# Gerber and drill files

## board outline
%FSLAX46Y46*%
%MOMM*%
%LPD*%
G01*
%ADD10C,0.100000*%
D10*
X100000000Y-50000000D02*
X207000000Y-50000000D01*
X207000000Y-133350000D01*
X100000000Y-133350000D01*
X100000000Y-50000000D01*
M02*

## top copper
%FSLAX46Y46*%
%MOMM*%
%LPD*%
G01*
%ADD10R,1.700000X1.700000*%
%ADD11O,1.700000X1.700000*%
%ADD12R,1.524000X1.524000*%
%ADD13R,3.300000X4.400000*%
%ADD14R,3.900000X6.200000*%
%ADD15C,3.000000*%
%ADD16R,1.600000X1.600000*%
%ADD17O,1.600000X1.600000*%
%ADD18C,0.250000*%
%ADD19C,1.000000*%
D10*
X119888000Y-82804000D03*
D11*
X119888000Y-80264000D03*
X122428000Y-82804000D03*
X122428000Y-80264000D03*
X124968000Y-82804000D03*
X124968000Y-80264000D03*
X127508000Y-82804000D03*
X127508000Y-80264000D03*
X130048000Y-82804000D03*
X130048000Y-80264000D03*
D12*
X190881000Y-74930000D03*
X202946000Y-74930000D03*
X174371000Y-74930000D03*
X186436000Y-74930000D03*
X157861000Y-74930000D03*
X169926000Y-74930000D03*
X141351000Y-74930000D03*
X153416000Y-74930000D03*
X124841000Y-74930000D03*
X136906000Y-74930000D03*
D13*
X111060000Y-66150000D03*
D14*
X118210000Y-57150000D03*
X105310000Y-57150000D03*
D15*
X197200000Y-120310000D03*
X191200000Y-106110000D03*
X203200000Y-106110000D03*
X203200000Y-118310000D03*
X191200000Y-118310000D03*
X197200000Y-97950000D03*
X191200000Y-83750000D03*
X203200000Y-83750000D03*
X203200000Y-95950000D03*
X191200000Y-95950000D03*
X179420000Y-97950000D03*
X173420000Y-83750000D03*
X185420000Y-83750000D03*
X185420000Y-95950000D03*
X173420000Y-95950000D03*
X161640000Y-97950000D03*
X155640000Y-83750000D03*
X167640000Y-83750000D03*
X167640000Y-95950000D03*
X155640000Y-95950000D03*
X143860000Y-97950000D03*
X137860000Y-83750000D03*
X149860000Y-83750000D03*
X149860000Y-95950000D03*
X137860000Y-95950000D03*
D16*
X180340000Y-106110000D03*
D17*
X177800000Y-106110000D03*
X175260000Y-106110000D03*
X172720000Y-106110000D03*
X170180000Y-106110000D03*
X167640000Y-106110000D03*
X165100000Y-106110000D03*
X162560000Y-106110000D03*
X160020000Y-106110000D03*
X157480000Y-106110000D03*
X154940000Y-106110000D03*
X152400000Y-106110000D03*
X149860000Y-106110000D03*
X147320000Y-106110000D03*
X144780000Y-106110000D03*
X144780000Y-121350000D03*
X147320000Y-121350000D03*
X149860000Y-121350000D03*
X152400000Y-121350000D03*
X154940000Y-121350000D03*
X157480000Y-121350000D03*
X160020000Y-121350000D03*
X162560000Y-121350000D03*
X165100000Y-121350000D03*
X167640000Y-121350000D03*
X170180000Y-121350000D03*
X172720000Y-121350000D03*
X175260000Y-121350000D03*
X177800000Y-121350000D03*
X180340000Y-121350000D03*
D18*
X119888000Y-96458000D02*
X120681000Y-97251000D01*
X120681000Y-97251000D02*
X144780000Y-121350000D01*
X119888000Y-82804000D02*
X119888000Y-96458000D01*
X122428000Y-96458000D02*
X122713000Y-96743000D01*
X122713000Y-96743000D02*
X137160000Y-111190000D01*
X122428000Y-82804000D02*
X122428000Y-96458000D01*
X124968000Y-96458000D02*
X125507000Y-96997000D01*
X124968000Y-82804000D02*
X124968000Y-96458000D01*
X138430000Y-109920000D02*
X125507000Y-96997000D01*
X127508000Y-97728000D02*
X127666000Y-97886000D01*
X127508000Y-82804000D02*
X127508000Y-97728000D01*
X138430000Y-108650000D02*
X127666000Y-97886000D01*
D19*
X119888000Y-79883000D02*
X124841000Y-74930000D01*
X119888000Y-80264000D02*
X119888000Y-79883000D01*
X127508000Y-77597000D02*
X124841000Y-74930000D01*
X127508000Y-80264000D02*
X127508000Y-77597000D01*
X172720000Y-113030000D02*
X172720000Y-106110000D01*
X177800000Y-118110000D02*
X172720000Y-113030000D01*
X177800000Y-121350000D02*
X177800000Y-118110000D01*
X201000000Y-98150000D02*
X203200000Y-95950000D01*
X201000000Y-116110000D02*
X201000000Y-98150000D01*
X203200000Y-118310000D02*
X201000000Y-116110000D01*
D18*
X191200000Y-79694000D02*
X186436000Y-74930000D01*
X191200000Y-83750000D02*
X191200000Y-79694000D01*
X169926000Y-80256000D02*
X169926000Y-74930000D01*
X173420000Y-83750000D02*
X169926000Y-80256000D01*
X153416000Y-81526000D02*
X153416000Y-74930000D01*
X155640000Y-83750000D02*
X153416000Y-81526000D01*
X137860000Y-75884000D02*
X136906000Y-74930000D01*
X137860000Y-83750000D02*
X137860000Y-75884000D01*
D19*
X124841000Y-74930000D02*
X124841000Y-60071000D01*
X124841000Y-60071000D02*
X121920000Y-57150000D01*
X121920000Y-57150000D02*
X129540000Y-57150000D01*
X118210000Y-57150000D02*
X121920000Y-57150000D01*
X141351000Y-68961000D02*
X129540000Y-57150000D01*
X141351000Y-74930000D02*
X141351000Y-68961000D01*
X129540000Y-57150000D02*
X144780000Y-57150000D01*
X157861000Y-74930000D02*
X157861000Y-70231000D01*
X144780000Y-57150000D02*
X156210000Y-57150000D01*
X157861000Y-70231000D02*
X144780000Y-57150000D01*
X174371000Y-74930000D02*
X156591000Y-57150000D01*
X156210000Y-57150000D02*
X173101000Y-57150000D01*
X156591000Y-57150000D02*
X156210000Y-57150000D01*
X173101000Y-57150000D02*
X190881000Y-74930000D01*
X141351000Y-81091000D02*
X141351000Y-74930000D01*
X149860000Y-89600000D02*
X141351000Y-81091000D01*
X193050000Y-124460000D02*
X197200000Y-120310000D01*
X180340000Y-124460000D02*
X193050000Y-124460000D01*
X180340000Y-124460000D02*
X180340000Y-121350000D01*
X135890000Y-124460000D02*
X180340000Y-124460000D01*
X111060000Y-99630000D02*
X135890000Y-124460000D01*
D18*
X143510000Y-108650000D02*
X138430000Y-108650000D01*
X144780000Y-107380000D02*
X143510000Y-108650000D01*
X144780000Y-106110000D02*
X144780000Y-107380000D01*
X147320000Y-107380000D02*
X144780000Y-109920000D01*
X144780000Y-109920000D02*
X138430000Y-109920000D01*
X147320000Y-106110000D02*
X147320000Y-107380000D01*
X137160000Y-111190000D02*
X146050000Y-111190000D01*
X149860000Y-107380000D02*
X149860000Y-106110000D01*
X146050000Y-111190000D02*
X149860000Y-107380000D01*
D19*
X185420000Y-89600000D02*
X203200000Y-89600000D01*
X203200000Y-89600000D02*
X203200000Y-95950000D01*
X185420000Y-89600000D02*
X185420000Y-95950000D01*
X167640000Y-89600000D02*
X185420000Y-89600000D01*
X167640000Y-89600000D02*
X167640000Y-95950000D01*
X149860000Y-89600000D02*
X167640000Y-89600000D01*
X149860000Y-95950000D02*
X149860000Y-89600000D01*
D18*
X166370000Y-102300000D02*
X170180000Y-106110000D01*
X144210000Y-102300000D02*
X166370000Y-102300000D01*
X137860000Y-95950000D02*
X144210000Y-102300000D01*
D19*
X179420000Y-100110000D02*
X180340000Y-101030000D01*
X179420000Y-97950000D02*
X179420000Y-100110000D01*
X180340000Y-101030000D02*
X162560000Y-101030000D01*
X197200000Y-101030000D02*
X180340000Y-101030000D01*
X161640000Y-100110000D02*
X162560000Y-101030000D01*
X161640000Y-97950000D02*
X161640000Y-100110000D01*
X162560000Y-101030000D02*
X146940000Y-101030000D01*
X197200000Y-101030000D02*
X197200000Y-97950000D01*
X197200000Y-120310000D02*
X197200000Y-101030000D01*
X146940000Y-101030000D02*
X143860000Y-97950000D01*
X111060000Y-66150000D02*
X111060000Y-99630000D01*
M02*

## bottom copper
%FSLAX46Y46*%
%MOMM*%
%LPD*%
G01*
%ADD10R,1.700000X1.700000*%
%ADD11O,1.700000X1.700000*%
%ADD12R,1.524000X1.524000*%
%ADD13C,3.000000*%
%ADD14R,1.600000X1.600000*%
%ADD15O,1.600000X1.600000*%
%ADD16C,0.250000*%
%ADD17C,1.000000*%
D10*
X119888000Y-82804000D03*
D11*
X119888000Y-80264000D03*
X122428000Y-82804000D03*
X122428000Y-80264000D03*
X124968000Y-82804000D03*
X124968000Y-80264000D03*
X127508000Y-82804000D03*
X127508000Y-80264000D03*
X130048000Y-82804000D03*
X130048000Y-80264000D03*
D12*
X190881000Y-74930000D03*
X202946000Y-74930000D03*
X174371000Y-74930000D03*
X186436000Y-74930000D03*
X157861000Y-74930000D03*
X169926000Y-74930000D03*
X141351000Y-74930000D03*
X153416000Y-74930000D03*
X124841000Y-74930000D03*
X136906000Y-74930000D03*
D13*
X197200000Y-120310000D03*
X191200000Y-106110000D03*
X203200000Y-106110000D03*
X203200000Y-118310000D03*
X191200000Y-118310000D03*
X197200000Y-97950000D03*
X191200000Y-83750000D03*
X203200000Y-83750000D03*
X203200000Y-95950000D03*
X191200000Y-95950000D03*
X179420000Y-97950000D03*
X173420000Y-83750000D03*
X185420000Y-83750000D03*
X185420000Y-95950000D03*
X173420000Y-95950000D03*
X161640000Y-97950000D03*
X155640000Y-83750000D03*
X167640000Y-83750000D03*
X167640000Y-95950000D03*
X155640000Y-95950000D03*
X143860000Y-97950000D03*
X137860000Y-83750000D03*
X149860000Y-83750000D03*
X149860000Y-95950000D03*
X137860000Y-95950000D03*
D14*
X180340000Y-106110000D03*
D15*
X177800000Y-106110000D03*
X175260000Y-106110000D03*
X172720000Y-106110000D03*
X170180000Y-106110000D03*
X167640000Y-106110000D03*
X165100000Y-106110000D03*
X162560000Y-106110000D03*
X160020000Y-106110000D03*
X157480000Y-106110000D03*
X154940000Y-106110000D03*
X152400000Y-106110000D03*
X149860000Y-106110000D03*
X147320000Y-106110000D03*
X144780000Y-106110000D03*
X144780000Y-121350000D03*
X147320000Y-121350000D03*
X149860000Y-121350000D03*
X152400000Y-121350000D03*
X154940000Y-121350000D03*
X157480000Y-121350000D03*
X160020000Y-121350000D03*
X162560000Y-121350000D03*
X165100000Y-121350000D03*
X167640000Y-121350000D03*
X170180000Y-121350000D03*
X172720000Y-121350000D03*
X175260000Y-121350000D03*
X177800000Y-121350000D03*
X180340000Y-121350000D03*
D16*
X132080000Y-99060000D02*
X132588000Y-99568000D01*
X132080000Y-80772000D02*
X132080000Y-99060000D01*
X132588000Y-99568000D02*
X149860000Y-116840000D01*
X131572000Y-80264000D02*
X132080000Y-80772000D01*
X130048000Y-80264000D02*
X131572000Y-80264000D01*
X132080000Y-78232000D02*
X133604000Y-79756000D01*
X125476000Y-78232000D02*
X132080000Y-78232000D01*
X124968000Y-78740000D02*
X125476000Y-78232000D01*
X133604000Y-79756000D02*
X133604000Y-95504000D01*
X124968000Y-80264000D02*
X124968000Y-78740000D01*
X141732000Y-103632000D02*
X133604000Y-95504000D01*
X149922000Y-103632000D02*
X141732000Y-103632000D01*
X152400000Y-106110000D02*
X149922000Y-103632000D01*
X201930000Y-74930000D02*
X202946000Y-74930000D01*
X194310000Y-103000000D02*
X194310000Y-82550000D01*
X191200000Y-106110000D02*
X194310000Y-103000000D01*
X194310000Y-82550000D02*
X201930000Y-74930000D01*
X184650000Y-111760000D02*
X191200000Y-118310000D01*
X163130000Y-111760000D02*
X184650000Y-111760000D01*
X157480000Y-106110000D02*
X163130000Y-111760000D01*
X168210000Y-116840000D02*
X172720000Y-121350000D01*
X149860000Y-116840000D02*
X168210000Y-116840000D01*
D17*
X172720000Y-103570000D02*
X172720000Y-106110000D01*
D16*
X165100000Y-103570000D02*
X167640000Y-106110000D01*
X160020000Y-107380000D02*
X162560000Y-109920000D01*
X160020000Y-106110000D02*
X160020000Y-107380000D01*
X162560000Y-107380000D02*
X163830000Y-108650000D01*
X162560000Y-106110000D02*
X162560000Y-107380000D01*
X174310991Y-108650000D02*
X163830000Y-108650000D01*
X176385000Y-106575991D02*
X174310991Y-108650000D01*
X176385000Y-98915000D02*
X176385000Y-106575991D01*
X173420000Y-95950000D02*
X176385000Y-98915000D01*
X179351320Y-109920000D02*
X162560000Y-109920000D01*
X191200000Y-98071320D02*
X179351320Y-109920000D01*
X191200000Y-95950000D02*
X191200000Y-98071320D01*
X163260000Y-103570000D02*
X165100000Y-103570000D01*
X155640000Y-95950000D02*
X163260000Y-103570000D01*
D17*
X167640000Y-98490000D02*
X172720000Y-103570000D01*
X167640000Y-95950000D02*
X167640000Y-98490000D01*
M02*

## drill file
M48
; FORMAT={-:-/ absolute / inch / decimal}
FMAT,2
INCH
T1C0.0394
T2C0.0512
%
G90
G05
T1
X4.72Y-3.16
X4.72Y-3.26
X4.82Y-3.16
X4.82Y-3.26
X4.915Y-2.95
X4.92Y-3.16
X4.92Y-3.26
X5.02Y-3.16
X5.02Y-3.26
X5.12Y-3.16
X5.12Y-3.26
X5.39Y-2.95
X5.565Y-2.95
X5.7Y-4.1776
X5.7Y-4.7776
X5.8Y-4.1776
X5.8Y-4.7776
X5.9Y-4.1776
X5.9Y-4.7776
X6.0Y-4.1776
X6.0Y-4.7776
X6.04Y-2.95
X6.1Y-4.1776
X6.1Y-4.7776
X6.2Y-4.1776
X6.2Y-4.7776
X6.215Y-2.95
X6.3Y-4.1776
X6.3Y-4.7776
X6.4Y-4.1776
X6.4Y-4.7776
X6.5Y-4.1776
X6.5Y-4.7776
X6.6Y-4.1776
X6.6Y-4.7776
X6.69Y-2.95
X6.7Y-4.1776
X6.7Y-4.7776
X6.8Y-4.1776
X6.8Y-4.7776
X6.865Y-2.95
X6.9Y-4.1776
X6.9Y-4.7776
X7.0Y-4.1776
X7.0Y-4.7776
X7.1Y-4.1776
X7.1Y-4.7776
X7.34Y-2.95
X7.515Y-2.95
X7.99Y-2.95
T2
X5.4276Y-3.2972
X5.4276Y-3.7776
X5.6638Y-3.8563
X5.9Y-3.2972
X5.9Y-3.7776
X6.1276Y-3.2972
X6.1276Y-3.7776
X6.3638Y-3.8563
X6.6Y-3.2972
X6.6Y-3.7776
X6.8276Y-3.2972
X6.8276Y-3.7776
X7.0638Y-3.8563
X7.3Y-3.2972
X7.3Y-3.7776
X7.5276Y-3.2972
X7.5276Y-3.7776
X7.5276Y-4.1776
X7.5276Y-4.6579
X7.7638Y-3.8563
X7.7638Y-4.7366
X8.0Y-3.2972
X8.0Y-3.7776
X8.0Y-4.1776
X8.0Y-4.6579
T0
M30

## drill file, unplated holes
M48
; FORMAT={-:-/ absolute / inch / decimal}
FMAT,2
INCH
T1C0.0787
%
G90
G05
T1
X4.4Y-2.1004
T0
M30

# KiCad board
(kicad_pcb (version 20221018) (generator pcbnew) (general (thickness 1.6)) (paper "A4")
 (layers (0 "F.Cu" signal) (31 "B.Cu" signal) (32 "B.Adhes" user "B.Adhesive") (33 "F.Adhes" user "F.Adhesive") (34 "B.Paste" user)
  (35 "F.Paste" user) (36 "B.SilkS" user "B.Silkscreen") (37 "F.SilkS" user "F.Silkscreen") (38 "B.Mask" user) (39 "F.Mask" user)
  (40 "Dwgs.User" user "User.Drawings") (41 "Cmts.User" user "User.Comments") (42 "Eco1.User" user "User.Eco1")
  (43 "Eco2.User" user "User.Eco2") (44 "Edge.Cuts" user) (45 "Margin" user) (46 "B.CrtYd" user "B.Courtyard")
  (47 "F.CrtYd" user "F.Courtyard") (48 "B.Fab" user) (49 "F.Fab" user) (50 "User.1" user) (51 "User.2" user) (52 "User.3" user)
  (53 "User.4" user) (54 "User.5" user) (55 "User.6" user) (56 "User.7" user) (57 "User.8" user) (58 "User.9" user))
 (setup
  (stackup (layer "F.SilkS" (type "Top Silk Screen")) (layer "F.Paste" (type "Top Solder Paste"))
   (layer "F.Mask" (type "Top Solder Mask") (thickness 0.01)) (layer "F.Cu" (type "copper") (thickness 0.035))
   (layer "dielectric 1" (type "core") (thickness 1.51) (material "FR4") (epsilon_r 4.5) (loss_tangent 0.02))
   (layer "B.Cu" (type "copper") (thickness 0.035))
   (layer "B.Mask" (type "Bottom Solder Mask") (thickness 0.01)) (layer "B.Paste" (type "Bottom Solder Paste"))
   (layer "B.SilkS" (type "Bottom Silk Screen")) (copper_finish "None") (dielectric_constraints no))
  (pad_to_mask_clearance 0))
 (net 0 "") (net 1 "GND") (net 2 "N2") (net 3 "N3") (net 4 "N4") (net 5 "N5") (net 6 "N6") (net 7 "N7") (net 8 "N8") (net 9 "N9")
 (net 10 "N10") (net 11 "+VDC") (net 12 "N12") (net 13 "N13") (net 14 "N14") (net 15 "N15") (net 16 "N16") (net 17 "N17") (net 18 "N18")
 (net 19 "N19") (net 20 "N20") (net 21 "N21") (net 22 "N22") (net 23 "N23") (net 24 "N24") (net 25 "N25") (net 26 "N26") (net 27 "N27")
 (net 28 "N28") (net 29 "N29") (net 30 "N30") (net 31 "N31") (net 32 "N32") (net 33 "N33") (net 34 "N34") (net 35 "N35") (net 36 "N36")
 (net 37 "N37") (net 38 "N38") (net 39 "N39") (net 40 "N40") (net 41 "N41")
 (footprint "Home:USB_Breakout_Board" (layer "F.Cu") (at 196.85 62.23)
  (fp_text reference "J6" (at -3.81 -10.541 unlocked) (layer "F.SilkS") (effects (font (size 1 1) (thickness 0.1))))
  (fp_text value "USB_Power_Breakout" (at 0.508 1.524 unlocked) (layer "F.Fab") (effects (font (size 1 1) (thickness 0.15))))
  (pad "1" thru_hole rect (at -5.969 12.7) (size 1.524 1.524) (drill 1) (layers "*.Cu" "*.Mask") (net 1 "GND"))
  (pad "2" thru_hole rect (at 6.096 12.7) (size 1.524 1.524) (drill 1) (layers "*.Cu" "*.Mask") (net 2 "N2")))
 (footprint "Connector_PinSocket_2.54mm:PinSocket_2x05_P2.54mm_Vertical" (layer "F.Cu") (at 119.888 80.264 90)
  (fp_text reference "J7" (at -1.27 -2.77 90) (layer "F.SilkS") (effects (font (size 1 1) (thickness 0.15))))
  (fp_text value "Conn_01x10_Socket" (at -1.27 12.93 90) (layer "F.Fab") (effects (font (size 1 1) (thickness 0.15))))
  (pad "1" thru_hole rect (at -2.54 0 90) (size 1.7 1.7) (drill 1) (layers "*.Cu" "*.Mask") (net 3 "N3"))
  (pad "2" thru_hole oval (at 0 0 90) (size 1.7 1.7) (drill 1) (layers "*.Cu" "*.Mask") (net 1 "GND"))
  (pad "3" thru_hole oval (at -2.54 2.54 90) (size 1.7 1.7) (drill 1) (layers "*.Cu" "*.Mask") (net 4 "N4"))
  (pad "4" thru_hole oval (at 0 2.54 90) (size 1.7 1.7) (drill 1) (layers "*.Cu" "*.Mask") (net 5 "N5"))
  (pad "5" thru_hole oval (at -2.54 5.08 90) (size 1.7 1.7) (drill 1) (layers "*.Cu" "*.Mask") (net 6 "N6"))
  (pad "6" thru_hole oval (at 0 5.08 90) (size 1.7 1.7) (drill 1) (layers "*.Cu" "*.Mask") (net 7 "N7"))
  (pad "7" thru_hole oval (at -2.54 7.62 90) (size 1.7 1.7) (drill 1) (layers "*.Cu" "*.Mask") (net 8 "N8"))
  (pad "8" thru_hole oval (at 0 7.62 90) (size 1.7 1.7) (drill 1) (layers "*.Cu" "*.Mask") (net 1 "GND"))
  (pad "9" thru_hole oval (at -2.54 10.16 90) (size 1.7 1.7) (drill 1) (layers "*.Cu" "*.Mask") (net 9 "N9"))
  (pad "10" thru_hole oval (at 0 10.16 90) (size 1.7 1.7) (drill 1) (layers "*.Cu" "*.Mask") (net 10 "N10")))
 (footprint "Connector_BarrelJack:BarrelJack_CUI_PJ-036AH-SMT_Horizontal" (layer "F.Cu") (at 111.76 60.35 180)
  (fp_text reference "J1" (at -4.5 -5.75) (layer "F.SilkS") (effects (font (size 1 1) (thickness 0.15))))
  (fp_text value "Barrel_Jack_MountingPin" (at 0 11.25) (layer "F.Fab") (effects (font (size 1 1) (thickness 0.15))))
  (pad "" np_thru_hole circle (at 0 7 180) (size 2 2) (drill 2) (layers "*.Cu" "*.Mask"))
  (pad "1" smd rect (at 0.7 -5.8 180) (size 3.3 4.4) (layers "F.Cu" "F.Paste" "F.Mask") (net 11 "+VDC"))
  (pad "2" smd rect (at -6.45 3.2 180) (size 3.9 6.2) (layers "F.Cu" "F.Paste" "F.Mask") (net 1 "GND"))
  (pad "3" smd rect (at 6.45 3.2 180) (size 3.9 6.2) (layers "F.Cu" "F.Paste" "F.Mask")))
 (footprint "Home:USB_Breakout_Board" (layer "F.Cu") (at 180.34 62.23)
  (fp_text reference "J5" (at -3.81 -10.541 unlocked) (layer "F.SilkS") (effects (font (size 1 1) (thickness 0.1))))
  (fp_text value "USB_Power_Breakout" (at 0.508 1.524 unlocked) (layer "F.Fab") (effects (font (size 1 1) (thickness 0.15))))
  (pad "1" thru_hole rect (at -5.969 12.7) (size 1.524 1.524) (drill 1) (layers "*.Cu" "*.Mask") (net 1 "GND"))
  (pad "2" thru_hole rect (at 6.096 12.7) (size 1.524 1.524) (drill 1) (layers "*.Cu" "*.Mask") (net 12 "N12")))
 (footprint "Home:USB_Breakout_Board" (layer "F.Cu") (at 130.81 62.23)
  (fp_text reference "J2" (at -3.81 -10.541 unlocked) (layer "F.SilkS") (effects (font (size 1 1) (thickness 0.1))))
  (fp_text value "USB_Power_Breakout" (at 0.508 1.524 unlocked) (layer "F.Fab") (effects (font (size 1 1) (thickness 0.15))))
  (pad "1" thru_hole rect (at -5.969 12.7) (size 1.524 1.524) (drill 1) (layers "*.Cu" "*.Mask") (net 1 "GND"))
  (pad "2" thru_hole rect (at 6.096 12.7) (size 1.524 1.524) (drill 1) (layers "*.Cu" "*.Mask") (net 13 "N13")))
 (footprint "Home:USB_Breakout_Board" (layer "F.Cu") (at 147.32 62.23)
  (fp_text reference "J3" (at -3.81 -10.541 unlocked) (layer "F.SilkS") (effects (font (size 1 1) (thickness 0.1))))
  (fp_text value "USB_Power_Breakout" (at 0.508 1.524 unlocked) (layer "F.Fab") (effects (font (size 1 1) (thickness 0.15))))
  (pad "1" thru_hole rect (at -5.969 12.7) (size 1.524 1.524) (drill 1) (layers "*.Cu" "*.Mask") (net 1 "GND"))
  (pad "2" thru_hole rect (at 6.096 12.7) (size 1.524 1.524) (drill 1) (layers "*.Cu" "*.Mask") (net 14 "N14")))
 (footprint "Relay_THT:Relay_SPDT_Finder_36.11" (layer "F.Cu") (at 161.64 97.95 90)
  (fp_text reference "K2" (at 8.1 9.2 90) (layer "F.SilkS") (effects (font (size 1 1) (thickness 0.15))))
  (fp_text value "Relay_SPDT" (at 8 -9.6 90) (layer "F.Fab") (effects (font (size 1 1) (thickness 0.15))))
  (pad "11" thru_hole circle (at 0 0 90) (size 3 3) (drill 1.3) (layers "*.Cu" "*.Mask") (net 11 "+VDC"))
  (pad "12" thru_hole circle (at 14.2 -6 90) (size 3 3) (drill 1.3) (layers "*.Cu" "*.Mask") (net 14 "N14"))
  (pad "14" thru_hole circle (at 14.2 6 90) (size 3 3) (drill 1.3) (layers "*.Cu" "*.Mask") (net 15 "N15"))
  (pad "A1" thru_hole circle (at 2 6 90) (size 3 3) (drill 1.3) (layers "*.Cu" "*.Mask") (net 1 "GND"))
  (pad "A2" thru_hole circle (at 2 -6 90) (size 3 3) (drill 1.3) (layers "*.Cu" "*.Mask") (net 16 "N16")))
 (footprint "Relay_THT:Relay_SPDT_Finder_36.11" (layer "F.Cu") (at 179.42 97.95 90)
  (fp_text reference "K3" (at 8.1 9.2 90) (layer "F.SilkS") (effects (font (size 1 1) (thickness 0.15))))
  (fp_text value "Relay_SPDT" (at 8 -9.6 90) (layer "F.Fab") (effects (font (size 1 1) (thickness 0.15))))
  (pad "11" thru_hole circle (at 0 0 90) (size 3 3) (drill 1.3) (layers "*.Cu" "*.Mask") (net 11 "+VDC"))
  (pad "12" thru_hole circle (at 14.2 -6 90) (size 3 3) (drill 1.3) (layers "*.Cu" "*.Mask") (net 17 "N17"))
  (pad "14" thru_hole circle (at 14.2 6 90) (size 3 3) (drill 1.3) (layers "*.Cu" "*.Mask") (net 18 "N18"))
  (pad "A1" thru_hole circle (at 2 6 90) (size 3 3) (drill 1.3) (layers "*.Cu" "*.Mask") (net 1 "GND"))
  (pad "A2" thru_hole circle (at 2 -6 90) (size 3 3) (drill 1.3) (layers "*.Cu" "*.Mask") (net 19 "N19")))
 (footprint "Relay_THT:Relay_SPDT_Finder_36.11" (layer "F.Cu") (at 197.2 97.95 90)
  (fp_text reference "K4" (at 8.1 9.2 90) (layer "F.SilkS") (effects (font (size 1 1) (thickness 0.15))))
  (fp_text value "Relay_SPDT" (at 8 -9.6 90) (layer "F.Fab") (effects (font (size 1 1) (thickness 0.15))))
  (pad "11" thru_hole circle (at 0 0 90) (size 3 3) (drill 1.3) (layers "*.Cu" "*.Mask") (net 11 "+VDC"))
  (pad "12" thru_hole circle (at 14.2 -6 90) (size 3 3) (drill 1.3) (layers "*.Cu" "*.Mask") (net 12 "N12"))
  (pad "14" thru_hole circle (at 14.2 6 90) (size 3 3) (drill 1.3) (layers "*.Cu" "*.Mask") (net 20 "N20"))
  (pad "A1" thru_hole circle (at 2 6 90) (size 3 3) (drill 1.3) (layers "*.Cu" "*.Mask") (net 1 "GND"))
  (pad "A2" thru_hole circle (at 2 -6 90) (size 3 3) (drill 1.3) (layers "*.Cu" "*.Mask") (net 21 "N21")))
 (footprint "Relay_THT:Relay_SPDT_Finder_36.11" (layer "F.Cu") (at 143.86 97.95 90)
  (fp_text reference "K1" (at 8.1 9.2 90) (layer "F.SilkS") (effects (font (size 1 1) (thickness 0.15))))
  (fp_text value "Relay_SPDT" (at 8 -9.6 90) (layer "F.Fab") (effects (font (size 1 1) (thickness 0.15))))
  (pad "11" thru_hole circle (at 0 0 90) (size 3 3) (drill 1.3) (layers "*.Cu" "*.Mask") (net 11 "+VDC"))
  (pad "12" thru_hole circle (at 14.2 -6 90) (size 3 3) (drill 1.3) (layers "*.Cu" "*.Mask") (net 13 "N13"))
  (pad "14" thru_hole circle (at 14.2 6 90) (size 3 3) (drill 1.3) (layers "*.Cu" "*.Mask") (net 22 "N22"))
  (pad "A1" thru_hole circle (at 2 6 90) (size 3 3) (drill 1.3) (layers "*.Cu" "*.Mask") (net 1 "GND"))
  (pad "A2" thru_hole circle (at 2 -6 90) (size 3 3) (drill 1.3) (layers "*.Cu" "*.Mask") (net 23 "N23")))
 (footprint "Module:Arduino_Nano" (layer "F.Cu") (at 180.34 106.11 -90)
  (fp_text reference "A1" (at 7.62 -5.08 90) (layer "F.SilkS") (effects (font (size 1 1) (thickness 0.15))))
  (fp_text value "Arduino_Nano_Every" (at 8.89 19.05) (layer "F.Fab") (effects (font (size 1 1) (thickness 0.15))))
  (pad "1" thru_hole rect (at 0 0 270) (size 1.6 1.6) (drill 1) (layers "*.Cu" "*.Mask") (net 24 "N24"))
  (pad "2" thru_hole oval (at 0 2.54 270) (size 1.6 1.6) (drill 1) (layers "*.Cu" "*.Mask") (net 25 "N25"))
  (pad "3" thru_hole oval (at 0 5.08 270) (size 1.6 1.6) (drill 1) (layers "*.Cu" "*.Mask") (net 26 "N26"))
  (pad "4" thru_hole oval (at 0 7.62 270) (size 1.6 1.6) (drill 1) (layers "*.Cu" "*.Mask") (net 1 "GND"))
  (pad "5" thru_hole oval (at 0 10.16 270) (size 1.6 1.6) (drill 1) (layers "*.Cu" "*.Mask") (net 23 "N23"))
  (pad "6" thru_hole oval (at 0 12.7 270) (size 1.6 1.6) (drill 1) (layers "*.Cu" "*.Mask") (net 16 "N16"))
  (pad "7" thru_hole oval (at 0 15.24 270) (size 1.6 1.6) (drill 1) (layers "*.Cu" "*.Mask") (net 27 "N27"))
  (pad "8" thru_hole oval (at 0 17.78 270) (size 1.6 1.6) (drill 1) (layers "*.Cu" "*.Mask") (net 19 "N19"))
  (pad "9" thru_hole oval (at 0 20.32 270) (size 1.6 1.6) (drill 1) (layers "*.Cu" "*.Mask") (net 21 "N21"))
  (pad "10" thru_hole oval (at 0 22.86 270) (size 1.6 1.6) (drill 1) (layers "*.Cu" "*.Mask") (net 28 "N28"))
  (pad "11" thru_hole oval (at 0 25.4 270) (size 1.6 1.6) (drill 1) (layers "*.Cu" "*.Mask") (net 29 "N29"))
  (pad "12" thru_hole oval (at 0 27.94 270) (size 1.6 1.6) (drill 1) (layers "*.Cu" "*.Mask") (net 7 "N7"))
  (pad "13" thru_hole oval (at 0 30.48 270) (size 1.6 1.6) (drill 1) (layers "*.Cu" "*.Mask") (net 4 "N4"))
  (pad "14" thru_hole oval (at 0 33.02 270) (size 1.6 1.6) (drill 1) (layers "*.Cu" "*.Mask") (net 6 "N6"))
  (pad "15" thru_hole oval (at 0 35.56 270) (size 1.6 1.6) (drill 1) (layers "*.Cu" "*.Mask") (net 8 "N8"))
  (pad "16" thru_hole oval (at 15.24 35.56 270) (size 1.6 1.6) (drill 1) (layers "*.Cu" "*.Mask") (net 3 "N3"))
  (pad "17" thru_hole oval (at 15.24 33.02 270) (size 1.6 1.6) (drill 1) (layers "*.Cu" "*.Mask") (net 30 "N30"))
  (pad "18" thru_hole oval (at 15.24 30.48 270) (size 1.6 1.6) (drill 1) (layers "*.Cu" "*.Mask") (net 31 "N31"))
  (pad "19" thru_hole oval (at 15.24 27.94 270) (size 1.6 1.6) (drill 1) (layers "*.Cu" "*.Mask") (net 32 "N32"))
  (pad "20" thru_hole oval (at 15.24 25.4 270) (size 1.6 1.6) (drill 1) (layers "*.Cu" "*.Mask") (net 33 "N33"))
  (pad "21" thru_hole oval (at 15.24 22.86 270) (size 1.6 1.6) (drill 1) (layers "*.Cu" "*.Mask") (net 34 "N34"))
  (pad "22" thru_hole oval (at 15.24 20.32 270) (size 1.6 1.6) (drill 1) (layers "*.Cu" "*.Mask") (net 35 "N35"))
  (pad "23" thru_hole oval (at 15.24 17.78 270) (size 1.6 1.6) (drill 1) (layers "*.Cu" "*.Mask") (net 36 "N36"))
  (pad "24" thru_hole oval (at 15.24 15.24 270) (size 1.6 1.6) (drill 1) (layers "*.Cu" "*.Mask") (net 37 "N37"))
  (pad "25" thru_hole oval (at 15.24 12.7 270) (size 1.6 1.6) (drill 1) (layers "*.Cu" "*.Mask") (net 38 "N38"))
  (pad "26" thru_hole oval (at 15.24 10.16 270) (size 1.6 1.6) (drill 1) (layers "*.Cu" "*.Mask") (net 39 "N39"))
  (pad "27" thru_hole oval (at 15.24 7.62 270) (size 1.6 1.6) (drill 1) (layers "*.Cu" "*.Mask") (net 10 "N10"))
  (pad "28" thru_hole oval (at 15.24 5.08 270) (size 1.6 1.6) (drill 1) (layers "*.Cu" "*.Mask") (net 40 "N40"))
  (pad "29" thru_hole oval (at 15.24 2.54 270) (size 1.6 1.6) (drill 1) (layers "*.Cu" "*.Mask") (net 1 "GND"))
  (pad "30" thru_hole oval (at 15.24 0 270) (size 1.6 1.6) (drill 1) (layers "*.Cu" "*.Mask") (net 11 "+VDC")))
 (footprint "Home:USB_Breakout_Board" (layer "F.Cu") (at 163.83 62.23)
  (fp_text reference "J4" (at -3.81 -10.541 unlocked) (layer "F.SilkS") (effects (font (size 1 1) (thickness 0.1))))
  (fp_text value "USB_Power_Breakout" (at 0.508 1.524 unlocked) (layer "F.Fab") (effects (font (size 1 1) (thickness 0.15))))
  (pad "1" thru_hole rect (at -5.969 12.7) (size 1.524 1.524) (drill 1) (layers "*.Cu" "*.Mask") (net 1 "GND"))
  (pad "2" thru_hole rect (at 6.096 12.7) (size 1.524 1.524) (drill 1) (layers "*.Cu" "*.Mask") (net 17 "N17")))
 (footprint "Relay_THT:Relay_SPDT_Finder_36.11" (layer "F.Cu") (at 197.2 120.31 90)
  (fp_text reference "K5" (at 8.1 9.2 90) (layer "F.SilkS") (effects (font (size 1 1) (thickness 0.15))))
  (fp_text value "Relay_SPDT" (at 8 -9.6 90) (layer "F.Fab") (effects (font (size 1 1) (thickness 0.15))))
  (pad "11" thru_hole circle (at 0 0 90) (size 3 3) (drill 1.3) (layers "*.Cu" "*.Mask") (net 11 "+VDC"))
  (pad "12" thru_hole circle (at 14.2 -6 90) (size 3 3) (drill 1.3) (layers "*.Cu" "*.Mask") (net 2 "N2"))
  (pad "14" thru_hole circle (at 14.2 6 90) (size 3 3) (drill 1.3) (layers "*.Cu" "*.Mask") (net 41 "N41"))
  (pad "A1" thru_hole circle (at 2 6 90) (size 3 3) (drill 1.3) (layers "*.Cu" "*.Mask") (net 1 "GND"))
  (pad "A2" thru_hole circle (at 2 -6 90) (size 3 3) (drill 1.3) (layers "*.Cu" "*.Mask") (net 28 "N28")))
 (gr_rect (start 100 50) (end 207 133.35) (stroke (width 0.1) (type default)) (fill none) (layer "Edge.Cuts"))
 (segment (start 201 98.15) (end 203.2 95.95) (width 1) (layer "F.Cu") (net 1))
 (segment (start 127.508 77.597) (end 124.841 74.93) (width 1) (layer "F.Cu") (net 1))
 (segment (start 127.508 80.264) (end 127.508 77.597) (width 1) (layer "F.Cu") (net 1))
 (segment (start 185.42 89.6) (end 185.42 95.95) (width 1) (layer "F.Cu") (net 1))
 (segment (start 157.861 74.93) (end 157.861 70.231) (width 1) (layer "F.Cu") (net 1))
 (segment (start 167.64 89.6) (end 185.42 89.6) (width 1) (layer "F.Cu") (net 1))
 (segment (start 119.888 80.264) (end 119.888 79.883) (width 1) (layer "F.Cu") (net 1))
 (segment (start 124.841 74.93) (end 124.841 60.071) (width 1) (layer "F.Cu") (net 1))
 (segment (start 121.92 57.15) (end 129.54 57.15) (width 1) (layer "F.Cu") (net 1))
 (segment (start 203.2 89.6) (end 203.2 95.95) (width 1) (layer "F.Cu") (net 1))
 (segment (start 174.371 74.93) (end 156.591 57.15) (width 1) (layer "F.Cu") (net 1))
 (segment (start 149.86 89.6) (end 167.64 89.6) (width 1) (layer "F.Cu") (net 1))
 (segment (start 129.54 57.15) (end 144.78 57.15) (width 1) (layer "F.Cu") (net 1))
 (segment (start 149.86 89.6) (end 141.351 81.091) (width 1) (layer "F.Cu") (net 1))
 (segment (start 201 116.11) (end 201 98.15) (width 1) (layer "F.Cu") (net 1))
 (segment (start 185.42 89.6) (end 203.2 89.6) (width 1) (layer "F.Cu") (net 1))
 (segment (start 149.86 95.95) (end 149.86 89.6) (width 1) (layer "F.Cu") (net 1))
 (segment (start 141.351 74.93) (end 141.351 68.961) (width 1) (layer "F.Cu") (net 1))
 (segment (start 167.64 89.6) (end 167.64 95.95) (width 1) (layer "F.Cu") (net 1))
 (segment (start 173.101 57.15) (end 190.881 74.93) (width 1) (layer "F.Cu") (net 1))
 (segment (start 177.8 118.11) (end 172.72 113.03) (width 1) (layer "F.Cu") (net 1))
 (segment (start 141.351 68.961) (end 129.54 57.15) (width 1) (layer "F.Cu") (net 1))
 (segment (start 119.888 79.883) (end 124.841 74.93) (width 1) (layer "F.Cu") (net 1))
 (segment (start 156.21 57.15) (end 173.101 57.15) (width 1) (layer "F.Cu") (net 1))
 (segment (start 124.841 60.071) (end 121.92 57.15) (width 1) (layer "F.Cu") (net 1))
 (segment (start 141.351 81.091) (end 141.351 74.93) (width 1) (layer "F.Cu") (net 1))
 (segment (start 177.8 121.35) (end 177.8 118.11) (width 1) (layer "F.Cu") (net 1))
 (segment (start 144.78 57.15) (end 156.21 57.15) (width 1) (layer "F.Cu") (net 1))
 (segment (start 203.2 118.31) (end 201 116.11) (width 1) (layer "F.Cu") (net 1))
 (segment (start 172.72 113.03) (end 172.72 106.11) (width 1) (layer "F.Cu") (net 1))
 (segment (start 118.21 57.15) (end 121.92 57.15) (width 1) (layer "F.Cu") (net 1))
 (segment (start 157.861 70.231) (end 144.78 57.15) (width 1) (layer "F.Cu") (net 1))
 (segment (start 156.591 57.15) (end 156.21 57.15) (width 1) (layer "F.Cu") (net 1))
 (segment (start 172.72 103.57) (end 172.72 106.11) (width 1) (layer "B.Cu") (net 1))
 (segment (start 167.64 95.95) (end 167.64 98.49) (width 1) (layer "B.Cu") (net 1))
 (segment (start 167.64 98.49) (end 172.72 103.57) (width 1) (layer "B.Cu") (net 1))
 (segment (start 144.21 102.3) (end 166.37 102.3) (width 0.25) (layer "F.Cu") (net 23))
 (segment (start 137.86 95.95) (end 144.21 102.3) (width 0.25) (layer "F.Cu") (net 23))
 (segment (start 166.37 102.3) (end 170.18 106.11) (width 0.25) (layer "F.Cu") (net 23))
 (segment (start 163.26 103.57) (end 165.1 103.57) (width 0.25) (layer "B.Cu") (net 16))
 (segment (start 165.1 103.57) (end 167.64 106.11) (width 0.25) (layer "B.Cu") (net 16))
 (segment (start 155.64 95.95) (end 163.26 103.57) (width 0.25) (layer "B.Cu") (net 16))
 (segment (start 173.42 95.95) (end 176.385 98.915) (width 0.25) (layer "B.Cu") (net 19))
 (segment (start 176.385 106.575991) (end 174.310991 108.65) (width 0.25) (layer "B.Cu") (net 19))
 (segment (start 162.56 107.38) (end 163.83 108.65) (width 0.25) (layer "B.Cu") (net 19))
 (segment (start 176.385 98.915) (end 176.385 106.575991) (width 0.25) (layer "B.Cu") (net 19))
 (segment (start 162.56 106.11) (end 162.56 107.38) (width 0.25) (layer "B.Cu") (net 19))
 (segment (start 174.310991 108.65) (end 163.83 108.65) (width 0.25) (layer "B.Cu") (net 19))
 (segment (start 179.35132 109.92) (end 162.56 109.92) (width 0.25) (layer "B.Cu") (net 21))
 (segment (start 191.2 95.95) (end 191.2 98.07132) (width 0.25) (layer "B.Cu") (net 21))
 (segment (start 191.2 98.07132) (end 179.35132 109.92) (width 0.25) (layer "B.Cu") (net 21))
 (segment (start 160.02 107.38) (end 162.56 109.92) (width 0.25) (layer "B.Cu") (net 21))
 (segment (start 160.02 106.11) (end 160.02 107.38) (width 0.25) (layer "B.Cu") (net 21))
 (segment (start 157.48 106.11) (end 163.13 111.76) (width 0.25) (layer "B.Cu") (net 28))
 (segment (start 163.13 111.76) (end 184.65 111.76) (width 0.25) (layer "B.Cu") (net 28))
 (segment (start 184.65 111.76) (end 191.2 118.31) (width 0.25) (layer "B.Cu") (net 28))
 (segment (start 124.968 78.74) (end 125.476 78.232) (width 0.25) (layer "B.Cu") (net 7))
 (segment (start 149.922 103.632) (end 141.732 103.632) (width 0.25) (layer "B.Cu") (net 7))
 (segment (start 132.08 78.232) (end 133.604 79.756) (width 0.25) (layer "B.Cu") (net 7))
 (segment (start 141.732 103.632) (end 133.604 95.504) (width 0.25) (layer "B.Cu") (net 7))
 (segment (start 133.604 79.756) (end 133.604 95.504) (width 0.25) (layer "B.Cu") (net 7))
 (segment (start 125.476 78.232) (end 132.08 78.232) (width 0.25) (layer "B.Cu") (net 7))
 (segment (start 152.4 106.11) (end 149.922 103.632) (width 0.25) (layer "B.Cu") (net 7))
 (segment (start 124.968 80.264) (end 124.968 78.74) (width 0.25) (layer "B.Cu") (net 7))
 (segment (start 122.428 82.804) (end 122.428 96.458) (width 0.25) (layer "F.Cu") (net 4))
 (segment (start 146.05 111.19) (end 149.86 107.38) (width 0.25) (layer "F.Cu") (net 4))
 (segment (start 122.428 96.458) (end 122.713 96.743) (width 0.25) (layer "F.Cu") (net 4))
 (segment (start 137.16 111.19) (end 146.05 111.19) (width 0.25) (layer "F.Cu") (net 4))
 (segment (start 122.713 96.743) (end 137.16 111.19) (width 0.25) (layer "F.Cu") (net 4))
 (segment (start 149.86 107.38) (end 149.86 106.11) (width 0.25) (layer "F.Cu") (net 4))
 (segment (start 138.43 109.92) (end 125.507 96.997) (width 0.25) (layer "F.Cu") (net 6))
 (segment (start 124.968 96.458) (end 125.507 96.997) (width 0.25) (layer "F.Cu") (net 6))
 (segment (start 124.968 82.804) (end 124.968 96.458) (width 0.25) (layer "F.Cu") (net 6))
 (segment (start 147.32 107.38) (end 144.78 109.92) (width 0.25) (layer "F.Cu") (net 6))
 (segment (start 147.32 106.11) (end 147.32 107.38) (width 0.25) (layer "F.Cu") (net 6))
 (segment (start 144.78 109.92) (end 138.43 109.92) (width 0.25) (layer "F.Cu") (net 6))
 (segment (start 127.508 82.804) (end 127.508 97.728) (width 0.25) (layer "F.Cu") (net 8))
 (segment (start 138.43 108.65) (end 127.666 97.886) (width 0.25) (layer "F.Cu") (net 8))
 (segment (start 127.508 97.728) (end 127.666 97.886) (width 0.25) (layer "F.Cu") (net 8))
 (segment (start 144.78 107.38) (end 143.51 108.65) (width 0.25) (layer "F.Cu") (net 8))
 (segment (start 143.51 108.65) (end 138.43 108.65) (width 0.25) (layer "F.Cu") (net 8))
 (segment (start 144.78 106.11) (end 144.78 107.38) (width 0.25) (layer "F.Cu") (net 8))
 (segment (start 119.888 82.804) (end 119.888 96.458) (width 0.25) (layer "F.Cu") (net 3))
 (segment (start 119.888 96.458) (end 120.681 97.251) (width 0.25) (layer "F.Cu") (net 3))
 (segment (start 120.681 97.251) (end 144.78 121.35) (width 0.25) (layer "F.Cu") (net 3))
 (segment (start 132.08 80.772) (end 132.08 99.06) (width 0.25) (layer "B.Cu") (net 10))
 (segment (start 130.048 80.264) (end 131.572 80.264) (width 0.25) (layer "B.Cu") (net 10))
 (segment (start 131.572 80.264) (end 132.08 80.772) (width 0.25) (layer "B.Cu") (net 10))
 (segment (start 168.21 116.84) (end 172.72 121.35) (width 0.25) (layer "B.Cu") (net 10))
 (segment (start 132.08 99.06) (end 132.588 99.568) (width 0.25) (layer "B.Cu") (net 10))
 (segment (start 149.86 116.84) (end 168.21 116.84) (width 0.25) (layer "B.Cu") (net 10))
 (segment (start 132.588 99.568) (end 149.86 116.84) (width 0.25) (layer "B.Cu") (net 10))
 (segment (start 197.2 101.03) (end 197.2 97.95) (width 1) (layer "F.Cu") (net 11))
 (segment (start 180.34 124.46) (end 193.05 124.46) (width 1) (layer "F.Cu") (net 11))
 (segment (start 162.56 101.03) (end 146.94 101.03) (width 1) (layer "F.Cu") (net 11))
 (segment (start 111.06 66.15) (end 111.06 99.63) (width 1) (layer "F.Cu") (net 11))
 (segment (start 179.42 97.95) (end 179.42 100.11) (width 1) (layer "F.Cu") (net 11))
 (segment (start 180.34 124.46) (end 180.34 121.35) (width 1) (layer "F.Cu") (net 11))
 (segment (start 135.89 124.46) (end 180.34 124.46) (width 1) (layer "F.Cu") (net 11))
 (segment (start 146.94 101.03) (end 143.86 97.95) (width 1) (layer "F.Cu") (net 11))
 (segment (start 197.2 120.31) (end 197.2 101.03) (width 1) (layer "F.Cu") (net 11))
 (segment (start 193.05 124.46) (end 197.2 120.31) (width 1) (layer "F.Cu") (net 11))
 (segment (start 180.34 101.03) (end 162.56 101.03) (width 1) (layer "F.Cu") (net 11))
 (segment (start 161.64 100.11) (end 162.56 101.03) (width 1) (layer "F.Cu") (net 11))
 (segment (start 179.42 100.11) (end 180.34 101.03) (width 1) (layer "F.Cu") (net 11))
 (segment (start 197.2 101.03) (end 180.34 101.03) (width 1) (layer "F.Cu") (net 11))
 (segment (start 161.64 97.95) (end 161.64 100.11) (width 1) (layer "F.Cu") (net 11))
 (segment (start 111.06 99.63) (end 135.89 124.46) (width 1) (layer "F.Cu") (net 11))
 (segment (start 137.86 83.75) (end 137.86 75.884) (width 0.25) (layer "F.Cu") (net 13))
 (segment (start 137.86 75.884) (end 136.906 74.93) (width 0.25) (layer "F.Cu") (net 13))
 (segment (start 155.64 83.75) (end 153.416 81.526) (width 0.25) (layer "F.Cu") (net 14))
 (segment (start 153.416 81.526) (end 153.416 74.93) (width 0.25) (layer "F.Cu") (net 14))
 (segment (start 173.42 83.75) (end 169.926 80.256) (width 0.25) (layer "F.Cu") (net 17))
 (segment (start 169.926 80.256) (end 169.926 74.93) (width 0.25) (layer "F.Cu") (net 17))
 (segment (start 191.2 83.75) (end 191.2 79.694) (width 0.25) (layer "F.Cu") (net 12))
 (segment (start 191.2 79.694) (end 186.436 74.93) (width 0.25) (layer "F.Cu") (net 12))
 (segment (start 194.31 82.55) (end 201.93 74.93) (width 0.25) (layer "B.Cu") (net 2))
 (segment (start 201.93 74.93) (end 202.946 74.93) (width 0.25) (layer "B.Cu") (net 2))
 (segment (start 194.31 103) (end 194.31 82.55) (width 0.25) (layer "B.Cu") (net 2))
 (segment (start 191.2 106.11) (end 194.31 103) (width 0.25) (layer "B.Cu") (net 2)))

